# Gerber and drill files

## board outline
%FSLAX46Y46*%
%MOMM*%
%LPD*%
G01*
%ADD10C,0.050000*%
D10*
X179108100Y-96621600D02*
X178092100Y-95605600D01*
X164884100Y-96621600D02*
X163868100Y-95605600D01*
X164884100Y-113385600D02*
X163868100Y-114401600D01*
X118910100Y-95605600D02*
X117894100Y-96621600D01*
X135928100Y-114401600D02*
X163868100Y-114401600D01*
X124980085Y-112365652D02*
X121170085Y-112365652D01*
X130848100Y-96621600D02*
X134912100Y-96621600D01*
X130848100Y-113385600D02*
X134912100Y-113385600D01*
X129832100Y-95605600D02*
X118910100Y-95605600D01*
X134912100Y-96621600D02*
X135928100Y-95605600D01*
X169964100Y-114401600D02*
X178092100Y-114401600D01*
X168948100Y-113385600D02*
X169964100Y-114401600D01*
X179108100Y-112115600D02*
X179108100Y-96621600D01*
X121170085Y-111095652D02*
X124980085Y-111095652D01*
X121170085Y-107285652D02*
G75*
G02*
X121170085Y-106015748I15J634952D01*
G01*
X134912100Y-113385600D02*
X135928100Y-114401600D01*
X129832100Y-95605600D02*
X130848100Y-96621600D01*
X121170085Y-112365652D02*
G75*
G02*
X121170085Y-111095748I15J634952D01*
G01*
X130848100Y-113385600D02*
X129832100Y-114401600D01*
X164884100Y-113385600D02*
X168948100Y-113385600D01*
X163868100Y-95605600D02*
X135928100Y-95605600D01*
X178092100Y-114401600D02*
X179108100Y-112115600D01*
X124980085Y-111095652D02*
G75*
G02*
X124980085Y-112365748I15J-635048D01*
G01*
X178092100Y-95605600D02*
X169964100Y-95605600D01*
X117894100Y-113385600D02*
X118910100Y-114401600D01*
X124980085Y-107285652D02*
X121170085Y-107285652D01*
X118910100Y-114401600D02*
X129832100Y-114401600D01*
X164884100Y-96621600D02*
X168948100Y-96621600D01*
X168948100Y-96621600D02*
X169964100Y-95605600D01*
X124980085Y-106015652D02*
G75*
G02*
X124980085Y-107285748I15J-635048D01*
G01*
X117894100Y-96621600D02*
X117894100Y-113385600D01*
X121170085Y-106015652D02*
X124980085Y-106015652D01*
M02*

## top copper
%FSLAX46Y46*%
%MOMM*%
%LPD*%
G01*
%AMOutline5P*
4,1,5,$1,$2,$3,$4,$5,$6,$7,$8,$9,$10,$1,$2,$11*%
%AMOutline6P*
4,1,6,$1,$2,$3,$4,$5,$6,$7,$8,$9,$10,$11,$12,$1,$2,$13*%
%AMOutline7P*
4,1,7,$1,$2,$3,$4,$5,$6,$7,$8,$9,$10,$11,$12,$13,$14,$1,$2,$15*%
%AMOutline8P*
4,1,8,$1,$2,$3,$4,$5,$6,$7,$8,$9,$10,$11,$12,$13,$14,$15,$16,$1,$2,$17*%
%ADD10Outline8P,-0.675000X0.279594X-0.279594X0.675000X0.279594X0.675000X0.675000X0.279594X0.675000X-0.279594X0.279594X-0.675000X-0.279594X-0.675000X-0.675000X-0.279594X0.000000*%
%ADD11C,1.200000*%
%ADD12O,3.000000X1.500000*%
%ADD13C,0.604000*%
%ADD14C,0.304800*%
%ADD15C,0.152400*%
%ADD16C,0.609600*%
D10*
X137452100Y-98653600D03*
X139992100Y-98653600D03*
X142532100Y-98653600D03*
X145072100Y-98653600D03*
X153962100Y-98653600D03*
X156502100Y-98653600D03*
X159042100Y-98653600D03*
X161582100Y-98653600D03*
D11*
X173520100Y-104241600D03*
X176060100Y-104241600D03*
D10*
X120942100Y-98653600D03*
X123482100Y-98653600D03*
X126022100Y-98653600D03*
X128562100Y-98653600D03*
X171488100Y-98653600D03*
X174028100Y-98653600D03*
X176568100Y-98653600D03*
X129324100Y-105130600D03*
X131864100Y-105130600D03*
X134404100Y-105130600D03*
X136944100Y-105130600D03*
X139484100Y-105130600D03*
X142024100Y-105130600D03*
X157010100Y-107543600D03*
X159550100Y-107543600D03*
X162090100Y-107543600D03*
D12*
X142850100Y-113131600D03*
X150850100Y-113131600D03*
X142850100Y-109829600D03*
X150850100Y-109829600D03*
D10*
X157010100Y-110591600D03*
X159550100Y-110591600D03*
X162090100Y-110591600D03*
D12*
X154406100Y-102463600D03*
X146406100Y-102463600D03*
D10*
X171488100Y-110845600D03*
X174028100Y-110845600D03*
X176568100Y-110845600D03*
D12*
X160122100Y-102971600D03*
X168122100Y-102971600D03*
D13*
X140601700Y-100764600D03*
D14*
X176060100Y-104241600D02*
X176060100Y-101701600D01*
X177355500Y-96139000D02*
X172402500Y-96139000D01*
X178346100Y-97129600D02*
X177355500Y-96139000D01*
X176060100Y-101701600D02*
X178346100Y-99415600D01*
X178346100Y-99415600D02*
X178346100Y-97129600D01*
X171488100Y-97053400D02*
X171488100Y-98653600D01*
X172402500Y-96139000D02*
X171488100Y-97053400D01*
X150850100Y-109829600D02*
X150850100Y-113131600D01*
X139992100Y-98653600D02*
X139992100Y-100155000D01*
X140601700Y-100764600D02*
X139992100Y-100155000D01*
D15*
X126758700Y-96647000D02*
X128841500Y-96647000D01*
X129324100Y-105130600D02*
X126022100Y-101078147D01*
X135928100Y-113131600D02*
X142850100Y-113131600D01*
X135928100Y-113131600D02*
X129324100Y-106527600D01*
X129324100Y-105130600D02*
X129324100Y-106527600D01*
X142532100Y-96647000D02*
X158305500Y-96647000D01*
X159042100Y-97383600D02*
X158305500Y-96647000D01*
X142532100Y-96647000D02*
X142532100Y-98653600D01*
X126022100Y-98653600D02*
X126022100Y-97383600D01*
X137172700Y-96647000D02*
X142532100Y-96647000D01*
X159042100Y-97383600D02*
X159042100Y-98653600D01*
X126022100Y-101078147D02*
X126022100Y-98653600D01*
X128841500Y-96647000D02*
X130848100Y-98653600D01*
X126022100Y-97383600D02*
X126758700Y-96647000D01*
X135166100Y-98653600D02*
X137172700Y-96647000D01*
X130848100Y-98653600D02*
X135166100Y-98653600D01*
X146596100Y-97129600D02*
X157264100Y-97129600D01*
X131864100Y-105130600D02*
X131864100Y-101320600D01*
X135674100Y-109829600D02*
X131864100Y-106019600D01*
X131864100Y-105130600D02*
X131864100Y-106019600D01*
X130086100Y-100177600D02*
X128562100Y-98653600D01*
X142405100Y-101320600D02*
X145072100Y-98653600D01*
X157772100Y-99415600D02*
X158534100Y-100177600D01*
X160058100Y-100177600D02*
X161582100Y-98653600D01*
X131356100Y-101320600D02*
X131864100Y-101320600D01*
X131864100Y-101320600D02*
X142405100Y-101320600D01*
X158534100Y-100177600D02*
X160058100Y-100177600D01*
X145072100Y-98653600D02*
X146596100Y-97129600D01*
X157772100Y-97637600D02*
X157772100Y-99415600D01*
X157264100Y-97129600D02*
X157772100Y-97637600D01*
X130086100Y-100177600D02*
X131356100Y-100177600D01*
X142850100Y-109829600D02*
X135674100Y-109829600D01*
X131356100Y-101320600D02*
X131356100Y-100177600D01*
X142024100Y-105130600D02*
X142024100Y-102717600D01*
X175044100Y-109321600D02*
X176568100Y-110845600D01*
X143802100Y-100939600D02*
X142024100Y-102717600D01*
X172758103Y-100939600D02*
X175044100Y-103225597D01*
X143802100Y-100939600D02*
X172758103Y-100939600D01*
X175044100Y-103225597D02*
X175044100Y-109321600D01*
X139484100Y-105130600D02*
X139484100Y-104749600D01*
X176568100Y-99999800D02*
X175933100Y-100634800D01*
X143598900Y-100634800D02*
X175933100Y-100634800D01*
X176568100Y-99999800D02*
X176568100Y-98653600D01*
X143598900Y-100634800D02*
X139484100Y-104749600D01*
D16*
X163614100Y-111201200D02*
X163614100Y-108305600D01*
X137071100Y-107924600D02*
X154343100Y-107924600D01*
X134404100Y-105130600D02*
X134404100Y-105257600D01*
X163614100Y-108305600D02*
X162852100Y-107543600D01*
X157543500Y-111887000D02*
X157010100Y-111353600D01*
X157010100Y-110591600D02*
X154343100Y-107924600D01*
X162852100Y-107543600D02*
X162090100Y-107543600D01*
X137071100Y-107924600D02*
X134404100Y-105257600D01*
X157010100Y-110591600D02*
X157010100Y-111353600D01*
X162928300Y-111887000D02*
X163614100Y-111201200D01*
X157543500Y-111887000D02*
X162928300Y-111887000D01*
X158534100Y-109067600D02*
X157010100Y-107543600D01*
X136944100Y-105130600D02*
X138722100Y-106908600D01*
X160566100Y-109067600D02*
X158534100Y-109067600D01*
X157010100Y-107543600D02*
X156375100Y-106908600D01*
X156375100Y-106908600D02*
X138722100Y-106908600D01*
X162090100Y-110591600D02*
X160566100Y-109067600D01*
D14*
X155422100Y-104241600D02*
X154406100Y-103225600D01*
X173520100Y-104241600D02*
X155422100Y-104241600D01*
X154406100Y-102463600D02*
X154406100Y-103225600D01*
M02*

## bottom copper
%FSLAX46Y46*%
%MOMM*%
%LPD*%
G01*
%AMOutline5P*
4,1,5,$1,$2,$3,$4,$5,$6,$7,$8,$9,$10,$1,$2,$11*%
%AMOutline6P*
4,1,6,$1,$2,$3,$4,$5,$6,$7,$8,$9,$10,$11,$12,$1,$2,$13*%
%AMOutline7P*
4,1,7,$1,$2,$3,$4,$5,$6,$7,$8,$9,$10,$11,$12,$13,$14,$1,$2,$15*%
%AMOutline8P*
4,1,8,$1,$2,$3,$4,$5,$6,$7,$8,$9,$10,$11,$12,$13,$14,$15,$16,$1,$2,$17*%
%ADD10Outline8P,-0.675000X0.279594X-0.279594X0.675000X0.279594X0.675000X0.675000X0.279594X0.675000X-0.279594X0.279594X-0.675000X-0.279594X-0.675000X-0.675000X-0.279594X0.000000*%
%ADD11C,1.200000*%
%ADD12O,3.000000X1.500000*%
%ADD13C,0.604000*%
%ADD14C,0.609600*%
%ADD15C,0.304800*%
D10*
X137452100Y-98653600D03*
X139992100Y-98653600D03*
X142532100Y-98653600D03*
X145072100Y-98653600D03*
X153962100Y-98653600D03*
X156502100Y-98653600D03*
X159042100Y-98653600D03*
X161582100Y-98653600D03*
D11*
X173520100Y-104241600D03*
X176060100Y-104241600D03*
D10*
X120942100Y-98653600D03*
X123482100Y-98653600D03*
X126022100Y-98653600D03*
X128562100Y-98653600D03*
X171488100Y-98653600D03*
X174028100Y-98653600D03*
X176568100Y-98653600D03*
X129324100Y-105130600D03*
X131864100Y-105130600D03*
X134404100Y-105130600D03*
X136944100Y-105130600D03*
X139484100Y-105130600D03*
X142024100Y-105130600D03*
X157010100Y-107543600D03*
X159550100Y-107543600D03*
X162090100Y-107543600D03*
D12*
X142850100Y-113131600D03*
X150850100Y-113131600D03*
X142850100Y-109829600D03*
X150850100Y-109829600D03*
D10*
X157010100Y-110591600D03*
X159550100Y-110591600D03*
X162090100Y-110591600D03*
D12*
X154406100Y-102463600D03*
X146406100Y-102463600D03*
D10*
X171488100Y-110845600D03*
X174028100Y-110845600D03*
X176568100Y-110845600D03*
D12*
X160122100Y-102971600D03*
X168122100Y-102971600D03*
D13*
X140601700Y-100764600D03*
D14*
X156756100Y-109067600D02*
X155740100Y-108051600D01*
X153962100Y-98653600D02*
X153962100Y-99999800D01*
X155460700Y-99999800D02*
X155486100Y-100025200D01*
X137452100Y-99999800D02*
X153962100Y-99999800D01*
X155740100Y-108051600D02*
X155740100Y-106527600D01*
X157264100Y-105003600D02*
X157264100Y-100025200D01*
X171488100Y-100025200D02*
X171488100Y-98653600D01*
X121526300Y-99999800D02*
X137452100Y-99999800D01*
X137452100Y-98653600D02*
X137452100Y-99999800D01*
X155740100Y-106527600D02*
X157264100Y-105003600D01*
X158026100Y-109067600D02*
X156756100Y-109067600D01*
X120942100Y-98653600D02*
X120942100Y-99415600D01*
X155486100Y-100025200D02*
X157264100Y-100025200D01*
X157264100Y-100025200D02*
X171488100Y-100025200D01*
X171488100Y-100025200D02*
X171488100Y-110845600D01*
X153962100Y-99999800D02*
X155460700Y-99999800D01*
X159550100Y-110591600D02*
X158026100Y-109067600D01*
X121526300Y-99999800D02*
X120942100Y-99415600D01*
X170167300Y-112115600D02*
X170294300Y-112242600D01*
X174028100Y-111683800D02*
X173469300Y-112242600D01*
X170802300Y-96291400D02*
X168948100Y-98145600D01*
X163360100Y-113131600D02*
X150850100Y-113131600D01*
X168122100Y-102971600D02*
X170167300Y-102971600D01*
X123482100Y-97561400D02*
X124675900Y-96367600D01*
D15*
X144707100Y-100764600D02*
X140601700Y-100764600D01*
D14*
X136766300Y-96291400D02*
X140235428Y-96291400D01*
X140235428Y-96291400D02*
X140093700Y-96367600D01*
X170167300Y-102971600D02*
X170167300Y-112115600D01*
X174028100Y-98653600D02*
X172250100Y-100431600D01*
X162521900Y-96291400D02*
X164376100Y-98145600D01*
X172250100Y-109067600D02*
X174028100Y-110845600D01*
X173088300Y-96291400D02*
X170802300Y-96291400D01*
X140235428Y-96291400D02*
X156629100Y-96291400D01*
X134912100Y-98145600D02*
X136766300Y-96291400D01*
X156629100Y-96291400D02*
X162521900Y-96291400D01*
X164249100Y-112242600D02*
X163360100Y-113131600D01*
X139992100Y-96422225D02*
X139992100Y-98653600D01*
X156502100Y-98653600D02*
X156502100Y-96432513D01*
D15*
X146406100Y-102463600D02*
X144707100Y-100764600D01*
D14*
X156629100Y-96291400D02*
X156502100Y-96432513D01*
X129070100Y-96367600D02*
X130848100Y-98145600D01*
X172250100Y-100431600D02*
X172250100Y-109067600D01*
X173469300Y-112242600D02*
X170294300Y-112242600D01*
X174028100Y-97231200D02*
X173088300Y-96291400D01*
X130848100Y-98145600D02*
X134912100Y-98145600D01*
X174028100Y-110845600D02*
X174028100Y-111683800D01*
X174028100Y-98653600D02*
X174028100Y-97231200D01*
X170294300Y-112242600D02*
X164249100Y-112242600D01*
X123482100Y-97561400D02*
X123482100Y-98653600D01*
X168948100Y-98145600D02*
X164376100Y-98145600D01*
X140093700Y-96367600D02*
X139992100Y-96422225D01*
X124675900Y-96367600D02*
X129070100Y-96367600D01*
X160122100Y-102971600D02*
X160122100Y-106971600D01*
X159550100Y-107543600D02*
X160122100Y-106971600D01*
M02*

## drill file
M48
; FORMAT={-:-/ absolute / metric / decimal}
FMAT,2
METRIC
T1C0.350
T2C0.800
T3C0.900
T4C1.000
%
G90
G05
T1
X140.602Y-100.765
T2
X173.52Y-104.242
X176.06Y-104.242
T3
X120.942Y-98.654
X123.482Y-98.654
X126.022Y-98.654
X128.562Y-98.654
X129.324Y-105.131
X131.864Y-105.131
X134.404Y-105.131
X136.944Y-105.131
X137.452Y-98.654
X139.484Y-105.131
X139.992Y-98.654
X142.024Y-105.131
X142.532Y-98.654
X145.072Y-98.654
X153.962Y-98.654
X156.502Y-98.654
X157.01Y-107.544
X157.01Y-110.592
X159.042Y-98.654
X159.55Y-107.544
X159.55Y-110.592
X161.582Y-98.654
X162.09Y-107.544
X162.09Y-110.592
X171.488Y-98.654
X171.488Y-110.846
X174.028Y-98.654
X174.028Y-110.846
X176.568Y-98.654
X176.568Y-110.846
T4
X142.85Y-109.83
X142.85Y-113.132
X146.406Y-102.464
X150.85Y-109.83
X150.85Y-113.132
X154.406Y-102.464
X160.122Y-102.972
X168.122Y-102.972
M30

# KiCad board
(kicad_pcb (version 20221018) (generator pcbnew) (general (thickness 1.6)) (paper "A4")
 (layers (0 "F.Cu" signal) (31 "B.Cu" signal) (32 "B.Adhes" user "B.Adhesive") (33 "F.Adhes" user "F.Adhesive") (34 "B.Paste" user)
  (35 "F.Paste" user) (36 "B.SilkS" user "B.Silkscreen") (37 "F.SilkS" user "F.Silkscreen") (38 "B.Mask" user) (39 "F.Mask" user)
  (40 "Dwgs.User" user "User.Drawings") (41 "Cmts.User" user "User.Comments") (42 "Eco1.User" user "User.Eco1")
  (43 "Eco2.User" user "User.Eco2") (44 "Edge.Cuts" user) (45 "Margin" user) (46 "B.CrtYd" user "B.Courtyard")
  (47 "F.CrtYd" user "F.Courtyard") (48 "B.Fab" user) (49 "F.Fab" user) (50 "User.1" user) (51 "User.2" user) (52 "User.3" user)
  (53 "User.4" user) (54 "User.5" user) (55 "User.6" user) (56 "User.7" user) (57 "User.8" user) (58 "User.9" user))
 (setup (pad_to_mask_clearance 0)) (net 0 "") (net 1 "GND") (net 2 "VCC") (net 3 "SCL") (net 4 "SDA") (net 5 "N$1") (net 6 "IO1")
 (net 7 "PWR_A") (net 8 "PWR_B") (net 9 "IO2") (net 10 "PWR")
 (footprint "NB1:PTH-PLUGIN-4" (layer "F.Cu") (at 137.4521 98.6536)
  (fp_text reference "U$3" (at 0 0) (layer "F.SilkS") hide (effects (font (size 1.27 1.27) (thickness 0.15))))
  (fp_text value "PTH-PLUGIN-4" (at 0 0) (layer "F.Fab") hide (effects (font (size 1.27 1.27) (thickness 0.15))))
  (pad "P1" thru_hole roundrect (at 0 0) (size 1.35 1.35) (drill 0.9) (layers "*.Cu" "*.Mask") (roundrect_rratio 0.25)
   (chamfer_ratio 0.2928932188) (chamfer top_left top_right bottom_left bottom_right) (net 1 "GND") (solder_mask_margin 0.0635)
   (thermal_bridge_angle 45))
  (pad "P2" thru_hole roundrect (at 2.54 0) (size 1.35 1.35) (drill 0.9) (layers "*.Cu" "*.Mask") (roundrect_rratio 0.25)
   (chamfer_ratio 0.2928932188) (chamfer top_left top_right bottom_left bottom_right) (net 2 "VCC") (solder_mask_margin 0.0635)
   (thermal_bridge_angle 45))
  (pad "P3" thru_hole roundrect (at 5.08 0) (size 1.35 1.35) (drill 0.9) (layers "*.Cu" "*.Mask") (roundrect_rratio 0.25)
   (chamfer_ratio 0.2928932188) (chamfer top_left top_right bottom_left bottom_right) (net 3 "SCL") (solder_mask_margin 0.0635)
   (thermal_bridge_angle 45))
  (pad "P4" thru_hole roundrect (at 7.62 0) (size 1.35 1.35) (drill 0.9) (layers "*.Cu" "*.Mask") (roundrect_rratio 0.25)
   (chamfer_ratio 0.2928932188) (chamfer top_left top_right bottom_left bottom_right) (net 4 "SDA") (solder_mask_margin 0.0635)
   (thermal_bridge_angle 45)))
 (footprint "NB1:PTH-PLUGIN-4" (layer "F.Cu") (at 153.9621 98.6536)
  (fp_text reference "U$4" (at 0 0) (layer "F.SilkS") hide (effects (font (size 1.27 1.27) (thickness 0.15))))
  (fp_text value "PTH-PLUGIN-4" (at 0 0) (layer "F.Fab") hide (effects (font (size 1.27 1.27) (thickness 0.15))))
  (pad "P1" thru_hole roundrect (at 0 0) (size 1.35 1.35) (drill 0.9) (layers "*.Cu" "*.Mask") (roundrect_rratio 0.25)
   (chamfer_ratio 0.2928932188) (chamfer top_left top_right bottom_left bottom_right) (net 1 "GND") (solder_mask_margin 0.0635)
   (thermal_bridge_angle 45))
  (pad "P2" thru_hole roundrect (at 2.54 0) (size 1.35 1.35) (drill 0.9) (layers "*.Cu" "*.Mask") (roundrect_rratio 0.25)
   (chamfer_ratio 0.2928932188) (chamfer top_left top_right bottom_left bottom_right) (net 2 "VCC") (solder_mask_margin 0.0635)
   (thermal_bridge_angle 45))
  (pad "P3" thru_hole roundrect (at 5.08 0) (size 1.35 1.35) (drill 0.9) (layers "*.Cu" "*.Mask") (roundrect_rratio 0.25)
   (chamfer_ratio 0.2928932188) (chamfer top_left top_right bottom_left bottom_right) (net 3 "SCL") (solder_mask_margin 0.0635)
   (thermal_bridge_angle 45))
  (pad "P4" thru_hole roundrect (at 7.62 0) (size 1.35 1.35) (drill 0.9) (layers "*.Cu" "*.Mask") (roundrect_rratio 0.25)
   (chamfer_ratio 0.2928932188) (chamfer top_left top_right bottom_left bottom_right) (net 4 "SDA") (solder_mask_margin 0.0635)
   (thermal_bridge_angle 45)))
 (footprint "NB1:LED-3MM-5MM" (layer "F.Cu") (at 174.7901 104.2416)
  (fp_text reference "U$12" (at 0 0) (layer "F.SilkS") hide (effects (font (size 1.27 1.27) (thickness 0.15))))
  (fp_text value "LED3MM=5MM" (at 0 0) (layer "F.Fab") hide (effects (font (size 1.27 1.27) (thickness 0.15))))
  (pad "A" thru_hole circle (at -1.27 0) (size 1.2 1.2) (drill 0.8) (layers "*.Cu" "*.Mask") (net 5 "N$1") (solder_mask_margin 0.0635))
  (pad "K" thru_hole circle (at 1.27 0) (size 1.2 1.2) (drill 0.8) (layers "*.Cu" "*.Mask") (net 1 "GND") (solder_mask_margin 0.0635)))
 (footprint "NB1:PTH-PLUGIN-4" (layer "F.Cu") (at 120.9421 98.6536)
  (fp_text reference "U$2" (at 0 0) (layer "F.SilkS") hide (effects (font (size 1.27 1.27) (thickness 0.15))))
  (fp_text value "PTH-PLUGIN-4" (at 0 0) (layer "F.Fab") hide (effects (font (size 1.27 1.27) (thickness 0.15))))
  (pad "P1" thru_hole roundrect (at 0 0) (size 1.35 1.35) (drill 0.9) (layers "*.Cu" "*.Mask") (roundrect_rratio 0.25)
   (chamfer_ratio 0.2928932188) (chamfer top_left top_right bottom_left bottom_right) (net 1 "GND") (solder_mask_margin 0.0635)
   (thermal_bridge_angle 45))
  (pad "P2" thru_hole roundrect (at 2.54 0) (size 1.35 1.35) (drill 0.9) (layers "*.Cu" "*.Mask") (roundrect_rratio 0.25)
   (chamfer_ratio 0.2928932188) (chamfer top_left top_right bottom_left bottom_right) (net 2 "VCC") (solder_mask_margin 0.0635)
   (thermal_bridge_angle 45))
  (pad "P3" thru_hole roundrect (at 5.08 0) (size 1.35 1.35) (drill 0.9) (layers "*.Cu" "*.Mask") (roundrect_rratio 0.25)
   (chamfer_ratio 0.2928932188) (chamfer top_left top_right bottom_left bottom_right) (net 3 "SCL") (solder_mask_margin 0.0635)
   (thermal_bridge_angle 45))
  (pad "P4" thru_hole roundrect (at 7.62 0) (size 1.35 1.35) (drill 0.9) (layers "*.Cu" "*.Mask") (roundrect_rratio 0.25)
   (chamfer_ratio 0.2928932188) (chamfer top_left top_right bottom_left bottom_right) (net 4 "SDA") (solder_mask_margin 0.0635)
   (thermal_bridge_angle 45)))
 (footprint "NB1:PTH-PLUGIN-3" (layer "F.Cu") (at 171.4881 98.6536)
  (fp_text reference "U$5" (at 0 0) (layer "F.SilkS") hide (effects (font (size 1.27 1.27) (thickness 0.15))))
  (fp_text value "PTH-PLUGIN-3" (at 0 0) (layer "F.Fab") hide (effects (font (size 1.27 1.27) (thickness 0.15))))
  (pad "P1" thru_hole roundrect (at 0 0) (size 1.35 1.35) (drill 0.9) (layers "*.Cu" "*.Mask") (roundrect_rratio 0.25)
   (chamfer_ratio 0.2928932188) (chamfer top_left top_right bottom_left bottom_right) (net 1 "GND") (solder_mask_margin 0.0635)
   (thermal_bridge_angle 45))
  (pad "P2" thru_hole roundrect (at 2.54 0) (size 1.35 1.35) (drill 0.9) (layers "*.Cu" "*.Mask") (roundrect_rratio 0.25)
   (chamfer_ratio 0.2928932188) (chamfer top_left top_right bottom_left bottom_right) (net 2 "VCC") (solder_mask_margin 0.0635)
   (thermal_bridge_angle 45))
  (pad "P3" thru_hole roundrect (at 5.08 0) (size 1.35 1.35) (drill 0.9) (layers "*.Cu" "*.Mask") (roundrect_rratio 0.25)
   (chamfer_ratio 0.2928932188) (chamfer top_left top_right bottom_left bottom_right) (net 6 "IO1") (solder_mask_margin 0.0635)
   (thermal_bridge_angle 45)))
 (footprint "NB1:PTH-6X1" (layer "F.Cu") (at 129.3241 105.1306)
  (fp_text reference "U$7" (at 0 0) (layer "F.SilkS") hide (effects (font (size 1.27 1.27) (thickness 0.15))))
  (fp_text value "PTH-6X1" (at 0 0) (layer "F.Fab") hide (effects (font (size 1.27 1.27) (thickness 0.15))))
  (pad "P1" thru_hole roundrect (at 0 0) (size 1.35 1.35) (drill 0.9) (layers "*.Cu" "*.Mask") (roundrect_rratio 0.25)
   (chamfer_ratio 0.2928932188) (chamfer top_left top_right bottom_left bottom_right) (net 3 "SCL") (solder_mask_margin 0.0635)
   (thermal_bridge_angle 45))
  (pad "P2" thru_hole roundrect (at 2.54 0) (size 1.35 1.35) (drill 0.9) (layers "*.Cu" "*.Mask") (roundrect_rratio 0.25)
   (chamfer_ratio 0.2928932188) (chamfer top_left top_right bottom_left bottom_right) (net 4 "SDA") (solder_mask_margin 0.0635)
   (thermal_bridge_angle 45))
  (pad "P3" thru_hole roundrect (at 5.08 0) (size 1.35 1.35) (drill 0.9) (layers "*.Cu" "*.Mask") (roundrect_rratio 0.25)
   (chamfer_ratio 0.2928932188) (chamfer top_left top_right bottom_left bottom_right) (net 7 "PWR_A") (solder_mask_margin 0.0635)
   (thermal_bridge_angle 45))
  (pad "P4" thru_hole roundrect (at 7.62 0) (size 1.35 1.35) (drill 0.9) (layers "*.Cu" "*.Mask") (roundrect_rratio 0.25)
   (chamfer_ratio 0.2928932188) (chamfer top_left top_right bottom_left bottom_right) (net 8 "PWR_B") (solder_mask_margin 0.0635)
   (thermal_bridge_angle 45))
  (pad "P5" thru_hole roundrect (at 10.16 0) (size 1.35 1.35) (drill 0.9) (layers "*.Cu" "*.Mask") (roundrect_rratio 0.25)
   (chamfer_ratio 0.2928932188) (chamfer top_left top_right bottom_left bottom_right) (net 6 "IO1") (solder_mask_margin 0.0635)
   (thermal_bridge_angle 45))
  (pad "P6" thru_hole roundrect (at 12.7 0) (size 1.35 1.35) (drill 0.9) (layers "*.Cu" "*.Mask") (roundrect_rratio 0.25)
   (chamfer_ratio 0.2928932188) (chamfer top_left top_right bottom_left bottom_right) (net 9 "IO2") (solder_mask_margin 0.0635)
   (thermal_bridge_angle 45)))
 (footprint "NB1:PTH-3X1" (layer "F.Cu") (at 157.0101 107.5436)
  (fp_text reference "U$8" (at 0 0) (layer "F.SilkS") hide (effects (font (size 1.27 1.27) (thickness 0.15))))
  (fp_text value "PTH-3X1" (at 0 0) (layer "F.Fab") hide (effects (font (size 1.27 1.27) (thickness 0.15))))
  (pad "P1" thru_hole roundrect (at 0 0) (size 1.35 1.35) (drill 0.9) (layers "*.Cu" "*.Mask") (roundrect_rratio 0.25)
   (chamfer_ratio 0.2928932188) (chamfer top_left top_right bottom_left bottom_right) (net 8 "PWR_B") (solder_mask_margin 0.0635)
   (thermal_bridge_angle 45))
  (pad "P2" thru_hole roundrect (at 2.54 0) (size 1.35 1.35) (drill 0.9) (layers "*.Cu" "*.Mask") (roundrect_rratio 0.25)
   (chamfer_ratio 0.2928932188) (chamfer top_left top_right bottom_left bottom_right) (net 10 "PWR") (solder_mask_margin 0.0635)
   (thermal_bridge_angle 45))
  (pad "P3" thru_hole roundrect (at 5.08 0) (size 1.35 1.35) (drill 0.9) (layers "*.Cu" "*.Mask") (roundrect_rratio 0.25)
   (chamfer_ratio 0.2928932188) (chamfer top_left top_right bottom_left bottom_right) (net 7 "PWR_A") (solder_mask_margin 0.0635)
   (thermal_bridge_angle 45)))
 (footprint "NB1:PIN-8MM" (layer "F.Cu") (at 146.8501 113.1316)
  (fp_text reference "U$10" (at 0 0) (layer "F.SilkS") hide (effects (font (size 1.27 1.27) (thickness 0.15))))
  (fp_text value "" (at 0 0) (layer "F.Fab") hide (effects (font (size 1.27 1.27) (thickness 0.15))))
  (pad "P1" thru_hole oval (at -4 0) (size 3 1.5) (drill 1) (layers "*.Cu" "*.Mask") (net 3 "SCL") (solder_mask_margin 0.0635)
   (thermal_bridge_angle 45))
  (pad "P2" thru_hole oval (at 4 0) (size 3 1.5) (drill 1) (layers "*.Cu" "*.Mask") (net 2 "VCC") (solder_mask_margin 0.0635)
   (thermal_bridge_angle 45)))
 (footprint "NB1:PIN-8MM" (layer "F.Cu") (at 146.8501 109.8296)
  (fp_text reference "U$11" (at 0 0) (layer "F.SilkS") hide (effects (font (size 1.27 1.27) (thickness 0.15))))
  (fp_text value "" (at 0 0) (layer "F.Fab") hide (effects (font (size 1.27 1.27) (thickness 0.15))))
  (pad "P1" thru_hole oval (at -4 0) (size 3 1.5) (drill 1) (layers "*.Cu" "*.Mask") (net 4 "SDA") (solder_mask_margin 0.0635)
   (thermal_bridge_angle 45))
  (pad "P2" thru_hole oval (at 4 0) (size 3 1.5) (drill 1) (layers "*.Cu" "*.Mask") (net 2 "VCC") (solder_mask_margin 0.0635)
   (thermal_bridge_angle 45)))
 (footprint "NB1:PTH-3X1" (layer "F.Cu") (at 157.0101 110.5916)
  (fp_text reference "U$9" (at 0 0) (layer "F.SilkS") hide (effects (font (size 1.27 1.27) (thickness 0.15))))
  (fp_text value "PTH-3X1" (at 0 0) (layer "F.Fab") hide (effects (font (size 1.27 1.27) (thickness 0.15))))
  (pad "P1" thru_hole roundrect (at 0 0) (size 1.35 1.35) (drill 0.9) (layers "*.Cu" "*.Mask") (roundrect_rratio 0.25)
   (chamfer_ratio 0.2928932188) (chamfer top_left top_right bottom_left bottom_right) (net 7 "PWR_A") (solder_mask_margin 0.0635)
   (thermal_bridge_angle 45))
  (pad "P2" thru_hole roundrect (at 2.54 0) (size 1.35 1.35) (drill 0.9) (layers "*.Cu" "*.Mask") (roundrect_rratio 0.25)
   (chamfer_ratio 0.2928932188) (chamfer top_left top_right bottom_left bottom_right) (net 1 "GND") (solder_mask_margin 0.0635)
   (thermal_bridge_angle 45))
  (pad "P3" thru_hole roundrect (at 5.08 0) (size 1.35 1.35) (drill 0.9) (layers "*.Cu" "*.Mask") (roundrect_rratio 0.25)
   (chamfer_ratio 0.2928932188) (chamfer top_left top_right bottom_left bottom_right) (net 8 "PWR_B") (solder_mask_margin 0.0635)
   (thermal_bridge_angle 45)))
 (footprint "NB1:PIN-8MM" (layer "F.Cu") (at 150.4061 102.4636 180)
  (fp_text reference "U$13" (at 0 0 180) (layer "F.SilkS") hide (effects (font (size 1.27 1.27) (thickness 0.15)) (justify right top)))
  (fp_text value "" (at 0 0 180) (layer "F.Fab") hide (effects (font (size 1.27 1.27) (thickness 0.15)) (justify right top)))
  (pad "P1" thru_hole oval (at -4 0 180) (size 3 1.5) (drill 1) (layers "*.Cu" "*.Mask") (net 5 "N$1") (solder_mask_margin 0.0635)
   (thermal_bridge_angle 45))
  (pad "P2" thru_hole oval (at 4 0 180) (size 3 1.5) (drill 1) (layers "*.Cu" "*.Mask") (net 2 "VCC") (solder_mask_margin 0.0635)
   (thermal_bridge_angle 45)))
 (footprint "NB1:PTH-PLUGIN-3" (layer "F.Cu") (at 171.4881 110.8456)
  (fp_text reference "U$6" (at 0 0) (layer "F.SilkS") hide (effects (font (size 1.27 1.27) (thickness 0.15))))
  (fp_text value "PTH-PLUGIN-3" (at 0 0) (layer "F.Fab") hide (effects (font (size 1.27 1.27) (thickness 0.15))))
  (pad "P1" thru_hole roundrect (at 0 0) (size 1.35 1.35) (drill 0.9) (layers "*.Cu" "*.Mask") (roundrect_rratio 0.25)
   (chamfer_ratio 0.2928932188) (chamfer top_left top_right bottom_left bottom_right) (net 1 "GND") (solder_mask_margin 0.0635)
   (thermal_bridge_angle 45))
  (pad "P2" thru_hole roundrect (at 2.54 0) (size 1.35 1.35) (drill 0.9) (layers "*.Cu" "*.Mask") (roundrect_rratio 0.25)
   (chamfer_ratio 0.2928932188) (chamfer top_left top_right bottom_left bottom_right) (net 2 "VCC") (solder_mask_margin 0.0635)
   (thermal_bridge_angle 45))
  (pad "P3" thru_hole roundrect (at 5.08 0) (size 1.35 1.35) (drill 0.9) (layers "*.Cu" "*.Mask") (roundrect_rratio 0.25)
   (chamfer_ratio 0.2928932188) (chamfer top_left top_right bottom_left bottom_right) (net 9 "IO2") (solder_mask_margin 0.0635)
   (thermal_bridge_angle 45)))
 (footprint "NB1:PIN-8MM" (layer "F.Cu") (at 164.1221 102.9716)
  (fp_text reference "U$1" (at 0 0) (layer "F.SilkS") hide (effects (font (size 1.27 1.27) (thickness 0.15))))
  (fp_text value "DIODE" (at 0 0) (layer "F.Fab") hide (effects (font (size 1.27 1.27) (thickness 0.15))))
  (pad "P1" thru_hole oval (at -4 0) (size 3 1.5) (drill 1) (layers "*.Cu" "*.Mask") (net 10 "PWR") (solder_mask_margin 0.0635)
   (thermal_bridge_angle 45))
  (pad "P2" thru_hole oval (at 4 0) (size 3 1.5) (drill 1) (layers "*.Cu" "*.Mask") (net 2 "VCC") (solder_mask_margin 0.0635)
   (thermal_bridge_angle 45)))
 (gr_line (start 179.1081 96.6216) (end 178.0921 95.6056) (stroke (width 0.05) (type solid)) (layer "Edge.Cuts"))
 (gr_line (start 164.8841 96.6216) (end 163.8681 95.6056) (stroke (width 0.05) (type solid)) (layer "Edge.Cuts"))
 (gr_line (start 164.8841 113.3856) (end 163.8681 114.4016) (stroke (width 0.05) (type solid)) (layer "Edge.Cuts"))
 (gr_line (start 118.9101 95.6056) (end 117.8941 96.6216) (stroke (width 0.05) (type solid)) (layer "Edge.Cuts"))
 (gr_line (start 135.9281 114.4016) (end 163.8681 114.4016) (stroke (width 0.05) (type solid)) (layer "Edge.Cuts"))
 (gr_line (start 124.980085 112.365652) (end 121.170085 112.365652) (stroke (width 0.05) (type default)) (layer "Edge.Cuts"))
 (gr_line (start 130.8481 96.6216) (end 134.9121 96.6216) (stroke (width 0.05) (type solid)) (layer "Edge.Cuts"))
 (gr_line (start 130.8481 113.3856) (end 134.9121 113.3856) (stroke (width 0.05) (type solid)) (layer "Edge.Cuts"))
 (gr_line (start 129.8321 95.6056) (end 118.9101 95.6056) (stroke (width 0.05) (type solid)) (layer "Edge.Cuts"))
 (gr_line (start 134.9121 96.6216) (end 135.9281 95.6056) (stroke (width 0.05) (type solid)) (layer "Edge.Cuts"))
 (gr_line (start 169.9641 114.4016) (end 178.0921 114.4016) (stroke (width 0.05) (type solid)) (layer "Edge.Cuts"))
 (gr_line (start 168.9481 113.3856) (end 169.9641 114.4016) (stroke (width 0.05) (type solid)) (layer "Edge.Cuts"))
 (gr_line (start 179.1081 112.1156) (end 179.1081 96.6216) (stroke (width 0.05) (type solid)) (layer "Edge.Cuts"))
 (gr_line (start 121.170085 111.095652) (end 124.980085 111.095652) (stroke (width 0.05) (type default)) (layer "Edge.Cuts"))
 (gr_arc (start 121.170085 107.285652) (mid 120.535085 106.650652) (end 121.170085 106.015652) (stroke (width 0.05) (type default))
  (layer "Edge.Cuts"))
 (gr_line (start 134.9121 113.3856) (end 135.9281 114.4016) (stroke (width 0.05) (type solid)) (layer "Edge.Cuts"))
 (gr_line (start 129.8321 95.6056) (end 130.8481 96.6216) (stroke (width 0.05) (type solid)) (layer "Edge.Cuts"))
 (gr_arc (start 121.170085 112.365652) (mid 120.535085 111.730652) (end 121.170085 111.095652) (stroke (width 0.05) (type default))
  (layer "Edge.Cuts"))
 (gr_line (start 130.8481 113.3856) (end 129.8321 114.4016) (stroke (width 0.05) (type solid)) (layer "Edge.Cuts"))
 (gr_line (start 164.8841 113.3856) (end 168.9481 113.3856) (stroke (width 0.05) (type solid)) (layer "Edge.Cuts"))
 (gr_line (start 163.8681 95.6056) (end 135.9281 95.6056) (stroke (width 0.05) (type solid)) (layer "Edge.Cuts"))
 (gr_line (start 178.0921 114.4016) (end 179.1081 112.1156) (stroke (width 0.05) (type solid)) (layer "Edge.Cuts"))
 (gr_arc (start 124.980085 111.095652) (mid 125.615085 111.730652) (end 124.980085 112.365652) (stroke (width 0.05) (type default))
  (layer "Edge.Cuts"))
 (gr_line (start 178.0921 95.6056) (end 169.9641 95.6056) (stroke (width 0.05) (type solid)) (layer "Edge.Cuts"))
 (gr_line (start 117.8941 113.3856) (end 118.9101 114.4016) (stroke (width 0.05) (type solid)) (layer "Edge.Cuts"))
 (gr_line (start 124.980085 107.285652) (end 121.170085 107.285652) (stroke (width 0.05) (type default)) (layer "Edge.Cuts"))
 (gr_line (start 118.9101 114.4016) (end 129.8321 114.4016) (stroke (width 0.05) (type solid)) (layer "Edge.Cuts"))
 (gr_line (start 164.8841 96.6216) (end 168.9481 96.6216) (stroke (width 0.05) (type solid)) (layer "Edge.Cuts"))
 (gr_line (start 168.9481 96.6216) (end 169.9641 95.6056) (stroke (width 0.05) (type solid)) (layer "Edge.Cuts"))
 (gr_arc (start 124.980085 106.015652) (mid 125.615085 106.650652) (end 124.980085 107.285652) (stroke (width 0.05) (type default))
  (layer "Edge.Cuts"))
 (gr_line (start 117.8941 96.6216) (end 117.8941 113.3856) (stroke (width 0.05) (type solid)) (layer "Edge.Cuts"))
 (gr_line (start 121.170085 106.015652) (end 124.980085 106.015652) (stroke (width 0.05) (type default)) (layer "Edge.Cuts"))
 (segment (start 176.0601 104.2416) (end 176.0601 101.7016) (width 0.3048) (layer "F.Cu") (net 1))
 (segment (start 177.3555 96.139) (end 172.4025 96.139) (width 0.3048) (layer "F.Cu") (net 1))
 (segment (start 178.3461 97.1296) (end 177.3555 96.139) (width 0.3048) (layer "F.Cu") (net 1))
 (segment (start 176.0601 101.7016) (end 178.3461 99.4156) (width 0.3048) (layer "F.Cu") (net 1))
 (segment (start 178.3461 99.4156) (end 178.3461 97.1296) (width 0.3048) (layer "F.Cu") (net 1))
 (segment (start 171.4881 97.0534) (end 171.4881 98.6536) (width 0.3048) (layer "F.Cu") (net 1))
 (segment (start 172.4025 96.139) (end 171.4881 97.0534) (width 0.3048) (layer "F.Cu") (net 1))
 (segment (start 156.7561 109.0676) (end 155.7401 108.0516) (width 0.6096) (layer "B.Cu") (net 1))
 (segment (start 153.9621 98.6536) (end 153.9621 99.9998) (width 0.6096) (layer "B.Cu") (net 1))
 (segment (start 155.4607 99.9998) (end 155.4861 100.0252) (width 0.6096) (layer "B.Cu") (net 1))
 (segment (start 137.4521 99.9998) (end 153.9621 99.9998) (width 0.6096) (layer "B.Cu") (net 1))
 (segment (start 155.7401 108.0516) (end 155.7401 106.5276) (width 0.6096) (layer "B.Cu") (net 1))
 (segment (start 157.2641 105.0036) (end 157.2641 100.0252) (width 0.6096) (layer "B.Cu") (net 1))
 (segment (start 171.4881 100.0252) (end 171.4881 98.6536) (width 0.6096) (layer "B.Cu") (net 1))
 (segment (start 121.5263 99.9998) (end 137.4521 99.9998) (width 0.6096) (layer "B.Cu") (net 1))
 (segment (start 137.4521 98.6536) (end 137.4521 99.9998) (width 0.6096) (layer "B.Cu") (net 1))
 (segment (start 155.7401 106.5276) (end 157.2641 105.0036) (width 0.6096) (layer "B.Cu") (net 1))
 (segment (start 158.0261 109.0676) (end 156.7561 109.0676) (width 0.6096) (layer "B.Cu") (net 1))
 (segment (start 120.9421 98.6536) (end 120.9421 99.4156) (width 0.6096) (layer "B.Cu") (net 1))
 (segment (start 155.4861 100.0252) (end 157.2641 100.0252) (width 0.6096) (layer "B.Cu") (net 1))
 (segment (start 157.2641 100.0252) (end 171.4881 100.0252) (width 0.6096) (layer "B.Cu") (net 1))
 (segment (start 171.4881 100.0252) (end 171.4881 110.8456) (width 0.6096) (layer "B.Cu") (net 1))
 (segment (start 153.9621 99.9998) (end 155.4607 99.9998) (width 0.6096) (layer "B.Cu") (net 1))
 (segment (start 159.5501 110.5916) (end 158.0261 109.0676) (width 0.6096) (layer "B.Cu") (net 1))
 (segment (start 121.5263 99.9998) (end 120.9421 99.4156) (width 0.6096) (layer "B.Cu") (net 1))
 (segment (start 150.8501 109.8296) (end 150.8501 113.1316) (width 0.3048) (layer "F.Cu") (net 2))
 (segment (start 139.9921 98.6536) (end 139.9921 100.155) (width 0.3048) (layer "F.Cu") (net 2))
 (segment (start 140.6017 100.7646) (end 139.9921 100.155) (width 0.3048) (layer "F.Cu") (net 2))
 (via (at 140.6017 100.7646) (size 0.604) (drill 0.35) (layers "F.Cu" "B.Cu") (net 2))
 (segment (start 170.1673 112.1156) (end 170.2943 112.2426) (width 0.6096) (layer "B.Cu") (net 2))
 (segment (start 174.0281 111.6838) (end 173.4693 112.2426) (width 0.6096) (layer "B.Cu") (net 2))
 (segment (start 170.8023 96.2914) (end 168.9481 98.1456) (width 0.6096) (layer "B.Cu") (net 2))
 (segment (start 163.3601 113.1316) (end 150.8501 113.1316) (width 0.6096) (layer "B.Cu") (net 2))
 (segment (start 168.1221 102.9716) (end 170.1673 102.9716) (width 0.6096) (layer "B.Cu") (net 2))
 (segment (start 123.4821 97.5614) (end 124.6759 96.3676) (width 0.6096) (layer "B.Cu") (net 2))
 (segment (start 144.7071 100.7646) (end 140.6017 100.7646) (width 0.3048) (layer "B.Cu") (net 2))
 (segment (start 136.7663 96.2914) (end 140.235428 96.2914) (width 0.6096) (layer "B.Cu") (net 2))
 (segment (start 140.235428 96.2914) (end 140.0937 96.3676) (width 0.6096) (layer "B.Cu") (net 2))
 (segment (start 170.1673 102.9716) (end 170.1673 112.1156) (width 0.6096) (layer "B.Cu") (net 2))
 (segment (start 174.0281 98.6536) (end 172.2501 100.4316) (width 0.6096) (layer "B.Cu") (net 2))
 (segment (start 162.5219 96.2914) (end 164.3761 98.1456) (width 0.6096) (layer "B.Cu") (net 2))
 (segment (start 172.2501 109.0676) (end 174.0281 110.8456) (width 0.6096) (layer "B.Cu") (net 2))
 (segment (start 173.0883 96.2914) (end 170.8023 96.2914) (width 0.6096) (layer "B.Cu") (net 2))
 (segment (start 140.235428 96.2914) (end 156.6291 96.2914) (width 0.6096) (layer "B.Cu") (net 2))
 (segment (start 134.9121 98.1456) (end 136.7663 96.2914) (width 0.6096) (layer "B.Cu") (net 2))
 (segment (start 156.6291 96.2914) (end 162.5219 96.2914) (width 0.6096) (layer "B.Cu") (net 2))
 (segment (start 164.2491 112.2426) (end 163.3601 113.1316) (width 0.6096) (layer "B.Cu") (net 2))
 (segment (start 139.9921 96.422225) (end 139.9921 98.6536) (width 0.6096) (layer "B.Cu") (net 2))
 (segment (start 156.5021 98.6536) (end 156.5021 96.432513) (width 0.6096) (layer "B.Cu") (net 2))
 (segment (start 146.4061 102.4636) (end 144.7071 100.7646) (width 0.3048) (layer "B.Cu") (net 2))
 (segment (start 156.6291 96.2914) (end 156.5021 96.432513) (width 0.6096) (layer "B.Cu") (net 2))
 (segment (start 129.0701 96.3676) (end 130.8481 98.1456) (width 0.6096) (layer "B.Cu") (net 2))
 (segment (start 172.2501 100.4316) (end 172.2501 109.0676) (width 0.6096) (layer "B.Cu") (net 2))
 (segment (start 173.4693 112.2426) (end 170.2943 112.2426) (width 0.6096) (layer "B.Cu") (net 2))
 (segment (start 174.0281 97.2312) (end 173.0883 96.2914) (width 0.6096) (layer "B.Cu") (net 2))
 (segment (start 130.8481 98.1456) (end 134.9121 98.1456) (width 0.6096) (layer "B.Cu") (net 2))
 (segment (start 174.0281 110.8456) (end 174.0281 111.6838) (width 0.6096) (layer "B.Cu") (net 2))
 (segment (start 174.0281 98.6536) (end 174.0281 97.2312) (width 0.6096) (layer "B.Cu") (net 2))
 (segment (start 170.2943 112.2426) (end 164.2491 112.2426) (width 0.6096) (layer "B.Cu") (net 2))
 (segment (start 123.4821 97.5614) (end 123.4821 98.6536) (width 0.6096) (layer "B.Cu") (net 2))
 (segment (start 168.9481 98.1456) (end 164.3761 98.1456) (width 0.6096) (layer "B.Cu") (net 2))
 (segment (start 140.0937 96.3676) (end 139.9921 96.422225) (width 0.6096) (layer "B.Cu") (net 2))
 (segment (start 124.6759 96.3676) (end 129.0701 96.3676) (width 0.6096) (layer "B.Cu") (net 2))
 (segment (start 126.7587 96.647) (end 128.8415 96.647) (width 0.1524) (layer "F.Cu") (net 3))
 (segment (start 129.3241 105.1306) (end 126.0221 101.078147) (width 0.1524) (layer "F.Cu") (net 3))
 (segment (start 135.9281 113.1316) (end 142.8501 113.1316) (width 0.1524) (layer "F.Cu") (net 3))
 (segment (start 135.9281 113.1316) (end 129.3241 106.5276) (width 0.1524) (layer "F.Cu") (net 3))
 (segment (start 129.3241 105.1306) (end 129.3241 106.5276) (width 0.1524) (layer "F.Cu") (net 3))
 (segment (start 142.5321 96.647) (end 158.3055 96.647) (width 0.1524) (layer "F.Cu") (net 3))
 (segment (start 159.0421 97.3836) (end 158.3055 96.647) (width 0.1524) (layer "F.Cu") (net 3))
 (segment (start 142.5321 96.647) (end 142.5321 98.6536) (width 0.1524) (layer "F.Cu") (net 3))
 (segment (start 126.0221 98.6536) (end 126.0221 97.3836) (width 0.1524) (layer "F.Cu") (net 3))
 (segment (start 137.1727 96.647) (end 142.5321 96.647) (width 0.1524) (layer "F.Cu") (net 3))
 (segment (start 159.0421 97.3836) (end 159.0421 98.6536) (width 0.1524) (layer "F.Cu") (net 3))
 (segment (start 126.0221 101.078147) (end 126.0221 98.6536) (width 0.1524) (layer "F.Cu") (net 3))
 (segment (start 128.8415 96.647) (end 130.8481 98.6536) (width 0.1524) (layer "F.Cu") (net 3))
 (segment (start 126.0221 97.3836) (end 126.7587 96.647) (width 0.1524) (layer "F.Cu") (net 3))
 (segment (start 135.1661 98.6536) (end 137.1727 96.647) (width 0.1524) (layer "F.Cu") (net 3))
 (segment (start 130.8481 98.6536) (end 135.1661 98.6536) (width 0.1524) (layer "F.Cu") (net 3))
 (segment (start 146.5961 97.1296) (end 157.2641 97.1296) (width 0.1524) (layer "F.Cu") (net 4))
 (segment (start 131.8641 105.1306) (end 131.8641 101.3206) (width 0.1524) (layer "F.Cu") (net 4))
 (segment (start 135.6741 109.8296) (end 131.8641 106.0196) (width 0.1524) (layer "F.Cu") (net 4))
 (segment (start 131.8641 105.1306) (end 131.8641 106.0196) (width 0.1524) (layer "F.Cu") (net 4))
 (segment (start 130.0861 100.1776) (end 128.5621 98.6536) (width 0.1524) (layer "F.Cu") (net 4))
 (segment (start 142.4051 101.3206) (end 145.0721 98.6536) (width 0.1524) (layer "F.Cu") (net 4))
 (segment (start 157.7721 99.4156) (end 158.5341 100.1776) (width 0.1524) (layer "F.Cu") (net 4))
 (segment (start 160.0581 100.1776) (end 161.5821 98.6536) (width 0.1524) (layer "F.Cu") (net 4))
 (segment (start 131.3561 101.3206) (end 131.8641 101.3206) (width 0.1524) (layer "F.Cu") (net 4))
 (segment (start 131.8641 101.3206) (end 142.4051 101.3206) (width 0.1524) (layer "F.Cu") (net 4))
 (segment (start 158.5341 100.1776) (end 160.0581 100.1776) (width 0.1524) (layer "F.Cu") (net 4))
 (segment (start 145.0721 98.6536) (end 146.5961 97.1296) (width 0.1524) (layer "F.Cu") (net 4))
 (segment (start 157.7721 97.6376) (end 157.7721 99.4156) (width 0.1524) (layer "F.Cu") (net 4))
 (segment (start 157.2641 97.1296) (end 157.7721 97.6376) (width 0.1524) (layer "F.Cu") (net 4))
 (segment (start 130.0861 100.1776) (end 131.3561 100.1776) (width 0.1524) (layer "F.Cu") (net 4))
 (segment (start 142.8501 109.8296) (end 135.6741 109.8296) (width 0.1524) (layer "F.Cu") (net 4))
 (segment (start 131.3561 101.3206) (end 131.3561 100.1776) (width 0.1524) (layer "F.Cu") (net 4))
 (segment (start 142.0241 105.1306) (end 142.0241 102.7176) (width 0.1524) (layer "F.Cu") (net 9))
 (segment (start 175.0441 109.3216) (end 176.5681 110.8456) (width 0.1524) (layer "F.Cu") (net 9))
 (segment (start 143.8021 100.9396) (end 142.0241 102.7176) (width 0.1524) (layer "F.Cu") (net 9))
 (segment (start 172.758103 100.9396) (end 175.0441 103.225597) (width 0.1524) (layer "F.Cu") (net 9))
 (segment (start 143.8021 100.9396) (end 172.758103 100.9396) (width 0.1524) (layer "F.Cu") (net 9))
 (segment (start 175.0441 103.225597) (end 175.0441 109.3216) (width 0.1524) (layer "F.Cu") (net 9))
 (segment (start 139.4841 105.1306) (end 139.4841 104.7496) (width 0.1524) (layer "F.Cu") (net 6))
 (segment (start 176.5681 99.9998) (end 175.9331 100.6348) (width 0.1524) (layer "F.Cu") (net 6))
 (segment (start 143.5989 100.6348) (end 175.9331 100.6348) (width 0.1524) (layer "F.Cu") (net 6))
 (segment (start 176.5681 99.9998) (end 176.5681 98.6536) (width 0.1524) (layer "F.Cu") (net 6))
 (segment (start 143.5989 100.6348) (end 139.4841 104.7496) (width 0.1524) (layer "F.Cu") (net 6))
 (segment (start 163.6141 111.2012) (end 163.6141 108.3056) (width 0.6096) (layer "F.Cu") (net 7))
 (segment (start 137.0711 107.9246) (end 154.3431 107.9246) (width 0.6096) (layer "F.Cu") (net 7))
 (segment (start 134.4041 105.1306) (end 134.4041 105.2576) (width 0.6096) (layer "F.Cu") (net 7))
 (segment (start 163.6141 108.3056) (end 162.8521 107.5436) (width 0.6096) (layer "F.Cu") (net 7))
 (segment (start 157.5435 111.887) (end 157.0101 111.3536) (width 0.6096) (layer "F.Cu") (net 7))
 (segment (start 157.0101 110.5916) (end 154.3431 107.9246) (width 0.6096) (layer "F.Cu") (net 7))
 (segment (start 162.8521 107.5436) (end 162.0901 107.5436) (width 0.6096) (layer "F.Cu") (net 7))
 (segment (start 137.0711 107.9246) (end 134.4041 105.2576) (width 0.6096) (layer "F.Cu") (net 7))
 (segment (start 157.0101 110.5916) (end 157.0101 111.3536) (width 0.6096) (layer "F.Cu") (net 7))
 (segment (start 162.9283 111.887) (end 163.6141 111.2012) (width 0.6096) (layer "F.Cu") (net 7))
 (segment (start 157.5435 111.887) (end 162.9283 111.887) (width 0.6096) (layer "F.Cu") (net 7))
 (segment (start 158.5341 109.0676) (end 157.0101 107.5436) (width 0.6096) (layer "F.Cu") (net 8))
 (segment (start 136.9441 105.1306) (end 138.7221 106.9086) (width 0.6096) (layer "F.Cu") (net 8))
 (segment (start 160.5661 109.0676) (end 158.5341 109.0676) (width 0.6096) (layer "F.Cu") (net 8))
 (segment (start 157.0101 107.5436) (end 156.3751 106.9086) (width 0.6096) (layer "F.Cu") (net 8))
 (segment (start 156.3751 106.9086) (end 138.7221 106.9086) (width 0.6096) (layer "F.Cu") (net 8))
 (segment (start 162.0901 110.5916) (end 160.5661 109.0676) (width 0.6096) (layer "F.Cu") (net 8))
 (segment (start 160.1221 102.9716) (end 160.1221 106.9716) (width 0.6096) (layer "B.Cu") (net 10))
 (segment (start 159.5501 107.5436) (end 160.1221 106.9716) (width 0.6096) (layer "B.Cu") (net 10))
 (segment (start 155.4221 104.2416) (end 154.4061 103.2256) (width 0.3048) (layer "F.Cu") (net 5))
 (segment (start 173.5201 104.2416) (end 155.4221 104.2416) (width 0.3048) (layer "F.Cu") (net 5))
 (segment (start 154.4061 102.4636) (end 154.4061 103.2256) (width 0.3048) (layer "F.Cu") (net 5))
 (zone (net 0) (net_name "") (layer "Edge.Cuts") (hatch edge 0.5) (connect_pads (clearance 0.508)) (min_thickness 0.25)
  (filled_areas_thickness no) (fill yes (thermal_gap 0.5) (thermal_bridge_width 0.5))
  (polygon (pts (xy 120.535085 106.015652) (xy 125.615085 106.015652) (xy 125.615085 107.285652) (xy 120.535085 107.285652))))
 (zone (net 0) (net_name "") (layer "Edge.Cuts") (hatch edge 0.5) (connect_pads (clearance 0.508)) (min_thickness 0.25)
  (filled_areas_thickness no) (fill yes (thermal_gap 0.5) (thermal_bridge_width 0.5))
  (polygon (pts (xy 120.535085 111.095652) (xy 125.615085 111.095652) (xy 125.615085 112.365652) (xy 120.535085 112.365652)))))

